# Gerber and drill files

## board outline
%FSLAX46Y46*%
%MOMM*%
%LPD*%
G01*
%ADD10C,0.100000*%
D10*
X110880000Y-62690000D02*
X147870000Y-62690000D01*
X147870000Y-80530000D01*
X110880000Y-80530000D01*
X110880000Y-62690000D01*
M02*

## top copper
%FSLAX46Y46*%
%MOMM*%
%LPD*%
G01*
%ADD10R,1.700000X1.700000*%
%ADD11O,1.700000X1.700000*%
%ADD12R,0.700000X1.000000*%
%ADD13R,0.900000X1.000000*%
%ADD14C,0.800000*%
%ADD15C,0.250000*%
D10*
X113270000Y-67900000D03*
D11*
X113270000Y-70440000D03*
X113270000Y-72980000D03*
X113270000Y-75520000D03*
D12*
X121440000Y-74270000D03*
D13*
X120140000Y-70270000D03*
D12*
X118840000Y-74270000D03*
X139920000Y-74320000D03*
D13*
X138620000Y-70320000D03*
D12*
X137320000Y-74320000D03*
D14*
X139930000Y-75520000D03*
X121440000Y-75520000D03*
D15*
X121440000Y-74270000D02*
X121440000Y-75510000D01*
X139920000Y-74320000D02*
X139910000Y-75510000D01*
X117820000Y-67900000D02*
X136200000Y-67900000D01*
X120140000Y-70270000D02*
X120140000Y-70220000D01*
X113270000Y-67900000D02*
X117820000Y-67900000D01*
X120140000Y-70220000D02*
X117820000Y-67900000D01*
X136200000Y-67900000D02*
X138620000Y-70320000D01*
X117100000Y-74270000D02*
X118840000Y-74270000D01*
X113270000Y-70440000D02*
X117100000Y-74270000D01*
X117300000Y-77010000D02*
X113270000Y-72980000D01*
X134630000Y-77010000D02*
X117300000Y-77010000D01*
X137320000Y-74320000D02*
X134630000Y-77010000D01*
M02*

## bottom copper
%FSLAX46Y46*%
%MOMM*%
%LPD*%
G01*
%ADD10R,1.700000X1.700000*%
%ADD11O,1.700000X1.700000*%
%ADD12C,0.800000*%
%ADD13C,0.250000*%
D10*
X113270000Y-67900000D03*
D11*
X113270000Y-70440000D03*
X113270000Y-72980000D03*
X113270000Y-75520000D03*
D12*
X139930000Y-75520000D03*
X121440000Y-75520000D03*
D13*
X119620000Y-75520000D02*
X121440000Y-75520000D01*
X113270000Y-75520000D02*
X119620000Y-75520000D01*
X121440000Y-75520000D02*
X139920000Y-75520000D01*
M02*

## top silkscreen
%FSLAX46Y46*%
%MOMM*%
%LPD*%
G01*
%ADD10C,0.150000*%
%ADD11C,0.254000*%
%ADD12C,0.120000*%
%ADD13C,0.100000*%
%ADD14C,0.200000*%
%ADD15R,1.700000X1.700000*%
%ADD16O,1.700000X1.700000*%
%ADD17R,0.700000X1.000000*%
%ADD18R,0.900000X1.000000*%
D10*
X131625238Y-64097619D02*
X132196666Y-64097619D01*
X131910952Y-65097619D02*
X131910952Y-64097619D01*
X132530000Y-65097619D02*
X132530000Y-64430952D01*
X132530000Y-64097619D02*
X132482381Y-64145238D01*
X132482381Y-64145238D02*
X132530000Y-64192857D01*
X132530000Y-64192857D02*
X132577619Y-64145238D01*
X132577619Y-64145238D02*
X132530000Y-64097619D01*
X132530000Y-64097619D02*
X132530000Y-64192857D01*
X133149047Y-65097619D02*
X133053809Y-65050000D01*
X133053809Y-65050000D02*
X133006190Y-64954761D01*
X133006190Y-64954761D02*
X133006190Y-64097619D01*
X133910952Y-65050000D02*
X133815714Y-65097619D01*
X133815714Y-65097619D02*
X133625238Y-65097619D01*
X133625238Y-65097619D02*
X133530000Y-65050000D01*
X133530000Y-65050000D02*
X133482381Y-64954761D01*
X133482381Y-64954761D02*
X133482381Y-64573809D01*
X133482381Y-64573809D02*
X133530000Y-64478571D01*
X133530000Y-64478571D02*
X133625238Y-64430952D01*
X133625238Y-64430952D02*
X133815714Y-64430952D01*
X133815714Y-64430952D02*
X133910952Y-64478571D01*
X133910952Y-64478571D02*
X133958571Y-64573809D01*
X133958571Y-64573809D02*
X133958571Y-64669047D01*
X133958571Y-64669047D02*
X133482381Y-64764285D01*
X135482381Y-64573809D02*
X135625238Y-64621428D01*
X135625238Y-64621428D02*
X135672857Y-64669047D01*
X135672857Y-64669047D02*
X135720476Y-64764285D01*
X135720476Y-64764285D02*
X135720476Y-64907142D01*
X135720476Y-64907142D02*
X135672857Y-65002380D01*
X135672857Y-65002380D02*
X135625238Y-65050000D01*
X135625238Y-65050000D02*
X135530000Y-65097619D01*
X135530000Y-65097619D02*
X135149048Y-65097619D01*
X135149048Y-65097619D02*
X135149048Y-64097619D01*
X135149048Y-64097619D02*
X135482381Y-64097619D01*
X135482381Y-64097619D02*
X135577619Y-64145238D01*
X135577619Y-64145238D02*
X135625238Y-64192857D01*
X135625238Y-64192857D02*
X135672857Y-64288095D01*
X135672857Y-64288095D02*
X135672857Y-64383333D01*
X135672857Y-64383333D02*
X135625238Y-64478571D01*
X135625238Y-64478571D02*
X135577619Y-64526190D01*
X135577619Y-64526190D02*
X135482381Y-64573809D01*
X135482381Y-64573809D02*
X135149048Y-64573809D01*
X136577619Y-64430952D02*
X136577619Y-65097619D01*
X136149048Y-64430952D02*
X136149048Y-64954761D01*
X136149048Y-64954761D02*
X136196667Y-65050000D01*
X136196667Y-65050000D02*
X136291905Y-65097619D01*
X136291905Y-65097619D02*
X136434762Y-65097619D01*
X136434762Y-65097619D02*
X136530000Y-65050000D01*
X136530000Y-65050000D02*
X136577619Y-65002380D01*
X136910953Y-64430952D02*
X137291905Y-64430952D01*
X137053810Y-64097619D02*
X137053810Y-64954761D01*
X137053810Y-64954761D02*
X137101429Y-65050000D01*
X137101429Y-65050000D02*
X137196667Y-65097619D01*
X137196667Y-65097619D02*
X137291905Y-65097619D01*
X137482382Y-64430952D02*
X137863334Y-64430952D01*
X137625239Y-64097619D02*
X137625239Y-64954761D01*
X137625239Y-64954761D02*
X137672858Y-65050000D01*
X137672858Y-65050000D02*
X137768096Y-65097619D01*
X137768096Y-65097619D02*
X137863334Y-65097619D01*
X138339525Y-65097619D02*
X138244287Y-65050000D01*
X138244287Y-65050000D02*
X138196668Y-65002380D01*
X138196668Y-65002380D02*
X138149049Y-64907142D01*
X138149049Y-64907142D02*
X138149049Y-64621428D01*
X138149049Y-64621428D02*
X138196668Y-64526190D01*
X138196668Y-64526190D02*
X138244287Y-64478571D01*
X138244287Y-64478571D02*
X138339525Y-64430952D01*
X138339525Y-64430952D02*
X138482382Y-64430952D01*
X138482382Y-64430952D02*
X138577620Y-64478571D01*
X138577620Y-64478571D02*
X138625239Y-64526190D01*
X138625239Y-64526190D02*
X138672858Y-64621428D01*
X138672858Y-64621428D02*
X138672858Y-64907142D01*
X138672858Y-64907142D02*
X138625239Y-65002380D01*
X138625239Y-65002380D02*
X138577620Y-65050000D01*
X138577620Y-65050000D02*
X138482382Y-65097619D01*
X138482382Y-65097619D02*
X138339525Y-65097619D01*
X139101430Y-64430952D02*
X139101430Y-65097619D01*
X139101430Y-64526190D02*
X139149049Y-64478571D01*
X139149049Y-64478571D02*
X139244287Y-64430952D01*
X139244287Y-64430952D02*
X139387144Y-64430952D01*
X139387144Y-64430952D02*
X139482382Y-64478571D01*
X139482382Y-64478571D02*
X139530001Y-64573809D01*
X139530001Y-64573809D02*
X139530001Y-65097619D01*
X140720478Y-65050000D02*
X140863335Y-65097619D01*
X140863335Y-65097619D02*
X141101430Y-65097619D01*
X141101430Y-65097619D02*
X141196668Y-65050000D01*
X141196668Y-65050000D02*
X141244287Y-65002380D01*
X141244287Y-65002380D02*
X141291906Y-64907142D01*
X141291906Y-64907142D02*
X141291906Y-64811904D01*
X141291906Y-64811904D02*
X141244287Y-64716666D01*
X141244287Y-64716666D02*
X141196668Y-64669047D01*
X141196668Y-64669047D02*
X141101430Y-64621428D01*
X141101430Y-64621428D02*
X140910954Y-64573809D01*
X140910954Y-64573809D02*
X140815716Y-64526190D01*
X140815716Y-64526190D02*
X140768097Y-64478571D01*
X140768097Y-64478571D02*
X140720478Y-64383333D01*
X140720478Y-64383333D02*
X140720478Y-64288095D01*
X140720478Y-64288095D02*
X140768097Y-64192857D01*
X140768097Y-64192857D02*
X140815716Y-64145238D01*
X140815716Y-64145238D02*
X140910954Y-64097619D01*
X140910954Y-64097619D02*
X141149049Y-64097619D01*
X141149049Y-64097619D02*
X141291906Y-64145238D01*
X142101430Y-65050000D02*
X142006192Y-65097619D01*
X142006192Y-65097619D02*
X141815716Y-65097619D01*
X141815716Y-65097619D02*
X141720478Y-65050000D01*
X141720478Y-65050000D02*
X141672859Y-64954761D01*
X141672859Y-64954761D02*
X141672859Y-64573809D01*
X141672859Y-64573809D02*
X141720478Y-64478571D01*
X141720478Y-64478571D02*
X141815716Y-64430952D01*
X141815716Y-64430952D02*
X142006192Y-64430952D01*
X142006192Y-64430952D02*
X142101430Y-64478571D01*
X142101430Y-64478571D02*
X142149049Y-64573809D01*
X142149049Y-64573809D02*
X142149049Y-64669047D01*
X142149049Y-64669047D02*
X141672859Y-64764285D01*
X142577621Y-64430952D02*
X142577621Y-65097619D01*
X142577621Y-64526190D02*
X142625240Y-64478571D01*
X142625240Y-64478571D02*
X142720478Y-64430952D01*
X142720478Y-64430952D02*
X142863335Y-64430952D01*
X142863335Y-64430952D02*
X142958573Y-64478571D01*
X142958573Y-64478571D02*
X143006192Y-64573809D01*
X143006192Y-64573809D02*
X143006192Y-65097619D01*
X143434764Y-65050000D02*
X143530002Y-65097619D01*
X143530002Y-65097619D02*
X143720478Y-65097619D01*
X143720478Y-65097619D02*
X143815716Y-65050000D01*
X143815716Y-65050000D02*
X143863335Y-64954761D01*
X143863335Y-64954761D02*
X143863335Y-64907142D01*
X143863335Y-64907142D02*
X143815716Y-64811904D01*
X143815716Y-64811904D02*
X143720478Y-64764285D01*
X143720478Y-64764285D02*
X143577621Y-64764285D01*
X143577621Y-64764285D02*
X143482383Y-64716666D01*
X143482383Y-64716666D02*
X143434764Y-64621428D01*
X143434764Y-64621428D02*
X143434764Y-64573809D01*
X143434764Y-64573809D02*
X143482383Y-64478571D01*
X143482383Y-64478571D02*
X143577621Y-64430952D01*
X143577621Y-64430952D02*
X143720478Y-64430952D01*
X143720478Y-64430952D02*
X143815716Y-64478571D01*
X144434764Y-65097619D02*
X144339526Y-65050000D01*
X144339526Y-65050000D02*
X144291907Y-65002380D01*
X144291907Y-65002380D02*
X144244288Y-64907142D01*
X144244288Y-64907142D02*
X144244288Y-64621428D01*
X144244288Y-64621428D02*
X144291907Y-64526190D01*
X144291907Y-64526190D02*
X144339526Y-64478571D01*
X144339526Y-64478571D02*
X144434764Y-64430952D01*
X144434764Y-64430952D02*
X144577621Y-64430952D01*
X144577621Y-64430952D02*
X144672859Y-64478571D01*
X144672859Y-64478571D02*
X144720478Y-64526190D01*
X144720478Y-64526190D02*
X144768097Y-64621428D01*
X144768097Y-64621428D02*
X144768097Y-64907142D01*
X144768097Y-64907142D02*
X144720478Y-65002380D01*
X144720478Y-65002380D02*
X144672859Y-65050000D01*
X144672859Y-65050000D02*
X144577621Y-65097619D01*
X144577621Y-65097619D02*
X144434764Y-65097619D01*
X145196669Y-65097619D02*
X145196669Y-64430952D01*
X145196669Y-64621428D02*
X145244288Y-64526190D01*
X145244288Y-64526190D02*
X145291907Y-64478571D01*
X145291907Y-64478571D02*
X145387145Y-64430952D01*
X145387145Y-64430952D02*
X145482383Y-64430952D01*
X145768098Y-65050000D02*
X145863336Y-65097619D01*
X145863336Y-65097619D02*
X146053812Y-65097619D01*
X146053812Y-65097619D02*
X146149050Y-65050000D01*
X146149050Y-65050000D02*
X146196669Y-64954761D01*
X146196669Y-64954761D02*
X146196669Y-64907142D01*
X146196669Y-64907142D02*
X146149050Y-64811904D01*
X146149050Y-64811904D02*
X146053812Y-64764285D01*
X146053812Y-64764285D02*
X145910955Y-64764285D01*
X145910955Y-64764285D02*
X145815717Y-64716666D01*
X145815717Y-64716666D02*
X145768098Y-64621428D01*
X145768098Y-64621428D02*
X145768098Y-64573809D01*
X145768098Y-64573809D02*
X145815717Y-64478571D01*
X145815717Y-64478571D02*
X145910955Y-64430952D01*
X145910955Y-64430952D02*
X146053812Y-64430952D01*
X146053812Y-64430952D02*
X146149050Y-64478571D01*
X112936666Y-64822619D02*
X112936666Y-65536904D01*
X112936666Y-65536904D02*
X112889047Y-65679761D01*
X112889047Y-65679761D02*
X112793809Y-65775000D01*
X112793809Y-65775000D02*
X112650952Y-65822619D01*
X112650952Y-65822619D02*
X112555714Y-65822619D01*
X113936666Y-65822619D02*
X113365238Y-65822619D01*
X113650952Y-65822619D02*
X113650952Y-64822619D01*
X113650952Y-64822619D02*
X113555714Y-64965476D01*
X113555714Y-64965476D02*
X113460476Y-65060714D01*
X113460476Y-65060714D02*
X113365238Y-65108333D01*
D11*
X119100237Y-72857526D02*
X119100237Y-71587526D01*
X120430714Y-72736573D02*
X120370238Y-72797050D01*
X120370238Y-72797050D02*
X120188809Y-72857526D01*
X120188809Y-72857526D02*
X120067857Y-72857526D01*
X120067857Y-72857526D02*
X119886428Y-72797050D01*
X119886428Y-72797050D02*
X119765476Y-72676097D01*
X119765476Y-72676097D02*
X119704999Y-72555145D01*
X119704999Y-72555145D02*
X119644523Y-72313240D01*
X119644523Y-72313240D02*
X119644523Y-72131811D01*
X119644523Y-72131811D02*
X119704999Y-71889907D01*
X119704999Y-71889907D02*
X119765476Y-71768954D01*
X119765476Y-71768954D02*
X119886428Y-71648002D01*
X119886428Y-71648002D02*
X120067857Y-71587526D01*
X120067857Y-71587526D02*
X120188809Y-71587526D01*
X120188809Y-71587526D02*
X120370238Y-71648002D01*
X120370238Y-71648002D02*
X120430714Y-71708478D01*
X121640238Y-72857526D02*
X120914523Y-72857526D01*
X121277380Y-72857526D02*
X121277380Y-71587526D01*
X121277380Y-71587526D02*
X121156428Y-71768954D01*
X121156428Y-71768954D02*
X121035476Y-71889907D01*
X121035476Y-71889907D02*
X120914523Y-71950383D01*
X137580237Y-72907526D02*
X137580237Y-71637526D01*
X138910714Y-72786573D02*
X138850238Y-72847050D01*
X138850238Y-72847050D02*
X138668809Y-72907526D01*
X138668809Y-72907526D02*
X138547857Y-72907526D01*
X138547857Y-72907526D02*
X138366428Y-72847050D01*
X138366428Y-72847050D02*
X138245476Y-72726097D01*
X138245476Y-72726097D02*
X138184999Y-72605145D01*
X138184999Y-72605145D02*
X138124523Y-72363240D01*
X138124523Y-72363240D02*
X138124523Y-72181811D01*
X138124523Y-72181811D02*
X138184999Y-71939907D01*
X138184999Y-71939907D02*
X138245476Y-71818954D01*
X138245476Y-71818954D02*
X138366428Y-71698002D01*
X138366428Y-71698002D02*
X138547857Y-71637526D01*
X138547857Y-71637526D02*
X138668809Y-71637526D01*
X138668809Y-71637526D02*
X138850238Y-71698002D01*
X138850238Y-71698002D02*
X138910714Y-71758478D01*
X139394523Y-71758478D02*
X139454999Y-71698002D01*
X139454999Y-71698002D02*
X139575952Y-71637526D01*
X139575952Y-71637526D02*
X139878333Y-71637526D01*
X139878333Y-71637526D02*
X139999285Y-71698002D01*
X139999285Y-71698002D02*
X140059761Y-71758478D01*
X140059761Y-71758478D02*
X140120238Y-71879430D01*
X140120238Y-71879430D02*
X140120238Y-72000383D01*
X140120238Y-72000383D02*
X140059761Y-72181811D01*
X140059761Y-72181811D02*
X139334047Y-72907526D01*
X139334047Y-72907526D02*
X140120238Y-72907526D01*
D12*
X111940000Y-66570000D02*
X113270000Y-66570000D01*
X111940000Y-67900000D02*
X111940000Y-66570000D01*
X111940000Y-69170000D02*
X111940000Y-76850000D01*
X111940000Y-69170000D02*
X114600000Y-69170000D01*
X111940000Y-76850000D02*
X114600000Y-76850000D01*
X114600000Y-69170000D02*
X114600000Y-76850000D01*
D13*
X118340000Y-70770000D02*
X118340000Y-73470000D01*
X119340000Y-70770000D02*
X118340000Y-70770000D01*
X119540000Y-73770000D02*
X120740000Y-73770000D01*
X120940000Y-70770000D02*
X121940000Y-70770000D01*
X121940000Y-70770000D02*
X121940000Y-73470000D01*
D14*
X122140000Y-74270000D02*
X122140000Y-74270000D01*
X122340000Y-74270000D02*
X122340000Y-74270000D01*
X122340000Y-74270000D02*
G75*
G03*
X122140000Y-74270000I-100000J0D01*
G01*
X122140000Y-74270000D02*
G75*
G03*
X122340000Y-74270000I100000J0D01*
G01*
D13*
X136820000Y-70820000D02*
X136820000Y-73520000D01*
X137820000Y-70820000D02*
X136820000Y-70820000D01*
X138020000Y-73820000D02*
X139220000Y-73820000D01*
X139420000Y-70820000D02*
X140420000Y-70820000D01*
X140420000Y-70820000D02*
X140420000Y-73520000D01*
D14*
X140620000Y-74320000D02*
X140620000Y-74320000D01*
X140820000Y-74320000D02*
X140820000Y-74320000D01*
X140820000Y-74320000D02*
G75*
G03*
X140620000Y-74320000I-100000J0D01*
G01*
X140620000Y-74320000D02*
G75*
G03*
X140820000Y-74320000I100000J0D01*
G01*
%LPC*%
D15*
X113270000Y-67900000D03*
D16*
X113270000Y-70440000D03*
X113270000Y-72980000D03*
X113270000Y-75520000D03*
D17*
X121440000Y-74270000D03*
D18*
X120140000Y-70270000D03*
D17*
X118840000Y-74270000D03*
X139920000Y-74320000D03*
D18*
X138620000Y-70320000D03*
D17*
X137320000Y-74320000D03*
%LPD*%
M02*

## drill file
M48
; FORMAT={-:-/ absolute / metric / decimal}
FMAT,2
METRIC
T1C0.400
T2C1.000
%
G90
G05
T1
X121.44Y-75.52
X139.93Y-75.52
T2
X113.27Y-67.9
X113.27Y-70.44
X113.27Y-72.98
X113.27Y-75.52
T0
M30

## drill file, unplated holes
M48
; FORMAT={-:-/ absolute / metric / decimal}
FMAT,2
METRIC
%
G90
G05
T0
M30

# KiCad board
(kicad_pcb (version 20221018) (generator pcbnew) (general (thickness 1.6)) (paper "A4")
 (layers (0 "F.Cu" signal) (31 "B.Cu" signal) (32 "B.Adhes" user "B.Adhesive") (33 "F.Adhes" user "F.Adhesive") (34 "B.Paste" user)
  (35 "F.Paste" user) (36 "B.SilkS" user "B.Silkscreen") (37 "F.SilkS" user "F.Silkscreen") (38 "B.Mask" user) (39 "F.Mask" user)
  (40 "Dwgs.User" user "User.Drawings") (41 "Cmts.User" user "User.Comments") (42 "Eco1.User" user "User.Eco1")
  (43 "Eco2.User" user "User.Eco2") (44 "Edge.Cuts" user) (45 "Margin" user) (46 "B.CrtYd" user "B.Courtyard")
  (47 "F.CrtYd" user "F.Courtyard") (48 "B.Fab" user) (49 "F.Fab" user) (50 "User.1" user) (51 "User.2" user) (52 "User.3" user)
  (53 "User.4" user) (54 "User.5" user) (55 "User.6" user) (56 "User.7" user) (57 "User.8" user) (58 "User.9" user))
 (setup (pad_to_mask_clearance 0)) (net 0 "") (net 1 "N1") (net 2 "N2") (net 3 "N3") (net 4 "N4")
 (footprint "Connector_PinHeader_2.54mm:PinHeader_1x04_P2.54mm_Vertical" (layer "F.Cu") (at 113.27 67.9)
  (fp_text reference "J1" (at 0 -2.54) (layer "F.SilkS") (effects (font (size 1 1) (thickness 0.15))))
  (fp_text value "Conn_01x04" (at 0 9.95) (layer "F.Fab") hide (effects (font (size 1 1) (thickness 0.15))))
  (fp_line (start -1.33 -1.33) (end 0 -1.33) (stroke (width 0.12) (type solid)) (layer "F.SilkS"))
  (fp_line (start -1.33 0) (end -1.33 -1.33) (stroke (width 0.12) (type solid)) (layer "F.SilkS"))
  (fp_line (start -1.33 1.27) (end -1.33 8.95) (stroke (width 0.12) (type solid)) (layer "F.SilkS"))
  (fp_line (start -1.33 1.27) (end 1.33 1.27) (stroke (width 0.12) (type solid)) (layer "F.SilkS"))
  (fp_line (start -1.33 8.95) (end 1.33 8.95) (stroke (width 0.12) (type solid)) (layer "F.SilkS"))
  (fp_line (start 1.33 1.27) (end 1.33 8.95) (stroke (width 0.12) (type solid)) (layer "F.SilkS"))
  (pad "GND" thru_hole rect (at 0 0) (size 1.7 1.7) (drill 1) (layers "*.Cu" "*.Mask") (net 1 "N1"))
  (pad "S1" thru_hole oval (at 0 2.54) (size 1.7 1.7) (drill 1) (layers "*.Cu" "*.Mask") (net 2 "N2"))
  (pad "S2" thru_hole oval (at 0 5.08) (size 1.7 1.7) (drill 1) (layers "*.Cu" "*.Mask") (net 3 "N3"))
  (pad "VCC" thru_hole oval (at 0 7.62) (size 1.7 1.7) (drill 1) (layers "*.Cu" "*.Mask") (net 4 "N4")))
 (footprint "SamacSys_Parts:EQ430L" (layer "F.Cu") (at 120.14 72.27)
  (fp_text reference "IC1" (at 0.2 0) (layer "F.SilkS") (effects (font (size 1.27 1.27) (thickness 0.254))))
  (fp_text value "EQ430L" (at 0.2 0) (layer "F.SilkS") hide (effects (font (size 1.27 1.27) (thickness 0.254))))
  (fp_line (start -1.8 -1.5) (end -1.8 1.2) (stroke (width 0.1) (type solid)) (layer "F.SilkS"))
  (fp_line (start -0.8 -1.5) (end -1.8 -1.5) (stroke (width 0.1) (type solid)) (layer "F.SilkS"))
  (fp_line (start -0.6 1.5) (end 0.6 1.5) (stroke (width 0.1) (type solid)) (layer "F.SilkS"))
  (fp_line (start 0.8 -1.5) (end 1.8 -1.5) (stroke (width 0.1) (type solid)) (layer "F.SilkS"))
  (fp_line (start 1.8 -1.5) (end 1.8 1.2) (stroke (width 0.1) (type solid)) (layer "F.SilkS"))
  (fp_line (start 2 2) (end 2 2) (stroke (width 0.2) (type solid)) (layer "F.SilkS"))
  (fp_line (start 2.2 2) (end 2.2 2) (stroke (width 0.2) (type solid)) (layer "F.SilkS"))
  (fp_arc (start 2 2) (mid 2.1 1.9) (end 2.2 2) (stroke (width 0.2) (type solid)) (layer "F.SilkS"))
  (fp_arc (start 2.2 2) (mid 2.1 2.1) (end 2 2) (stroke (width 0.2) (type solid)) (layer "F.SilkS"))
  (pad "1" smd rect (at 1.3 2) (size 0.7 1) (layers "F.Cu" "F.Paste" "F.Mask") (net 4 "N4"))
  (pad "2" smd rect (at 0 -2) (size 0.9 1) (layers "F.Cu" "F.Paste" "F.Mask") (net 1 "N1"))
  (pad "3" smd rect (at -1.3 2) (size 0.7 1) (layers "F.Cu" "F.Paste" "F.Mask") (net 2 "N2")))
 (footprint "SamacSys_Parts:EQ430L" (layer "F.Cu") (at 138.62 72.32)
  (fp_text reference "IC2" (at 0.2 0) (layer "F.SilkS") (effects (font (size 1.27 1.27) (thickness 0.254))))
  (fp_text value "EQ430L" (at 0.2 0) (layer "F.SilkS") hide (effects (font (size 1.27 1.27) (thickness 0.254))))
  (fp_line (start -1.8 -1.5) (end -1.8 1.2) (stroke (width 0.1) (type solid)) (layer "F.SilkS"))
  (fp_line (start -0.8 -1.5) (end -1.8 -1.5) (stroke (width 0.1) (type solid)) (layer "F.SilkS"))
  (fp_line (start -0.6 1.5) (end 0.6 1.5) (stroke (width 0.1) (type solid)) (layer "F.SilkS"))
  (fp_line (start 0.8 -1.5) (end 1.8 -1.5) (stroke (width 0.1) (type solid)) (layer "F.SilkS"))
  (fp_line (start 1.8 -1.5) (end 1.8 1.2) (stroke (width 0.1) (type solid)) (layer "F.SilkS"))
  (fp_line (start 2 2) (end 2 2) (stroke (width 0.2) (type solid)) (layer "F.SilkS"))
  (fp_line (start 2.2 2) (end 2.2 2) (stroke (width 0.2) (type solid)) (layer "F.SilkS"))
  (fp_arc (start 2 2) (mid 2.1 1.9) (end 2.2 2) (stroke (width 0.2) (type solid)) (layer "F.SilkS"))
  (fp_arc (start 2.2 2) (mid 2.1 2.1) (end 2 2) (stroke (width 0.2) (type solid)) (layer "F.SilkS"))
  (pad "1" smd rect (at 1.3 2) (size 0.7 1) (layers "F.Cu" "F.Paste" "F.Mask") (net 4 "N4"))
  (pad "2" smd rect (at 0 -2) (size 0.9 1) (layers "F.Cu" "F.Paste" "F.Mask") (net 1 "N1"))
  (pad "3" smd rect (at -1.3 2) (size 0.7 1) (layers "F.Cu" "F.Paste" "F.Mask") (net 3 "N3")))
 (gr_rect (start 110.88 62.69) (end 147.87 80.53) (stroke (width 0.1) (type default)) (fill none) (layer "Edge.Cuts"))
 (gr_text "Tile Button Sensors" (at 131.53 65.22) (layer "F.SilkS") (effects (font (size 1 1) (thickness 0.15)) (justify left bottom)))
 (segment (start 121.44 74.27) (end 121.44 75.51) (width 0.25) (layer "F.Cu") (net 4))
 (segment (start 139.92 74.32) (end 139.91 75.51) (width 0.25) (layer "F.Cu") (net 4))
 (via (at 139.93 75.52) (size 0.8) (drill 0.4) (layers "F.Cu" "B.Cu") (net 4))
 (via (at 121.44 75.52) (size 0.8) (drill 0.4) (layers "F.Cu" "B.Cu") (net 4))
 (segment (start 119.62 75.52) (end 121.44 75.52) (width 0.25) (layer "B.Cu") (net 4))
 (segment (start 113.27 75.52) (end 119.62 75.52) (width 0.25) (layer "B.Cu") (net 4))
 (segment (start 121.44 75.52) (end 139.92 75.52) (width 0.25) (layer "B.Cu") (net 4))
 (segment (start 117.82 67.9) (end 136.2 67.9) (width 0.25) (layer "F.Cu") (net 1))
 (segment (start 120.14 70.27) (end 120.14 70.22) (width 0.25) (layer "F.Cu") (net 1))
 (segment (start 113.27 67.9) (end 117.82 67.9) (width 0.25) (layer "F.Cu") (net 1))
 (segment (start 120.14 70.22) (end 117.82 67.9) (width 0.25) (layer "F.Cu") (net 1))
 (segment (start 136.2 67.9) (end 138.62 70.32) (width 0.25) (layer "F.Cu") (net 1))
 (segment (start 117.1 74.27) (end 118.84 74.27) (width 0.25) (layer "F.Cu") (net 2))
 (segment (start 113.27 70.44) (end 117.1 74.27) (width 0.25) (layer "F.Cu") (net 2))
 (segment (start 117.3 77.01) (end 113.27 72.98) (width 0.25) (layer "F.Cu") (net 3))
 (segment (start 134.63 77.01) (end 117.3 77.01) (width 0.25) (layer "F.Cu") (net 3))
 (segment (start 137.32 74.32) (end 134.63 77.01) (width 0.25) (layer "F.Cu") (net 3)))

